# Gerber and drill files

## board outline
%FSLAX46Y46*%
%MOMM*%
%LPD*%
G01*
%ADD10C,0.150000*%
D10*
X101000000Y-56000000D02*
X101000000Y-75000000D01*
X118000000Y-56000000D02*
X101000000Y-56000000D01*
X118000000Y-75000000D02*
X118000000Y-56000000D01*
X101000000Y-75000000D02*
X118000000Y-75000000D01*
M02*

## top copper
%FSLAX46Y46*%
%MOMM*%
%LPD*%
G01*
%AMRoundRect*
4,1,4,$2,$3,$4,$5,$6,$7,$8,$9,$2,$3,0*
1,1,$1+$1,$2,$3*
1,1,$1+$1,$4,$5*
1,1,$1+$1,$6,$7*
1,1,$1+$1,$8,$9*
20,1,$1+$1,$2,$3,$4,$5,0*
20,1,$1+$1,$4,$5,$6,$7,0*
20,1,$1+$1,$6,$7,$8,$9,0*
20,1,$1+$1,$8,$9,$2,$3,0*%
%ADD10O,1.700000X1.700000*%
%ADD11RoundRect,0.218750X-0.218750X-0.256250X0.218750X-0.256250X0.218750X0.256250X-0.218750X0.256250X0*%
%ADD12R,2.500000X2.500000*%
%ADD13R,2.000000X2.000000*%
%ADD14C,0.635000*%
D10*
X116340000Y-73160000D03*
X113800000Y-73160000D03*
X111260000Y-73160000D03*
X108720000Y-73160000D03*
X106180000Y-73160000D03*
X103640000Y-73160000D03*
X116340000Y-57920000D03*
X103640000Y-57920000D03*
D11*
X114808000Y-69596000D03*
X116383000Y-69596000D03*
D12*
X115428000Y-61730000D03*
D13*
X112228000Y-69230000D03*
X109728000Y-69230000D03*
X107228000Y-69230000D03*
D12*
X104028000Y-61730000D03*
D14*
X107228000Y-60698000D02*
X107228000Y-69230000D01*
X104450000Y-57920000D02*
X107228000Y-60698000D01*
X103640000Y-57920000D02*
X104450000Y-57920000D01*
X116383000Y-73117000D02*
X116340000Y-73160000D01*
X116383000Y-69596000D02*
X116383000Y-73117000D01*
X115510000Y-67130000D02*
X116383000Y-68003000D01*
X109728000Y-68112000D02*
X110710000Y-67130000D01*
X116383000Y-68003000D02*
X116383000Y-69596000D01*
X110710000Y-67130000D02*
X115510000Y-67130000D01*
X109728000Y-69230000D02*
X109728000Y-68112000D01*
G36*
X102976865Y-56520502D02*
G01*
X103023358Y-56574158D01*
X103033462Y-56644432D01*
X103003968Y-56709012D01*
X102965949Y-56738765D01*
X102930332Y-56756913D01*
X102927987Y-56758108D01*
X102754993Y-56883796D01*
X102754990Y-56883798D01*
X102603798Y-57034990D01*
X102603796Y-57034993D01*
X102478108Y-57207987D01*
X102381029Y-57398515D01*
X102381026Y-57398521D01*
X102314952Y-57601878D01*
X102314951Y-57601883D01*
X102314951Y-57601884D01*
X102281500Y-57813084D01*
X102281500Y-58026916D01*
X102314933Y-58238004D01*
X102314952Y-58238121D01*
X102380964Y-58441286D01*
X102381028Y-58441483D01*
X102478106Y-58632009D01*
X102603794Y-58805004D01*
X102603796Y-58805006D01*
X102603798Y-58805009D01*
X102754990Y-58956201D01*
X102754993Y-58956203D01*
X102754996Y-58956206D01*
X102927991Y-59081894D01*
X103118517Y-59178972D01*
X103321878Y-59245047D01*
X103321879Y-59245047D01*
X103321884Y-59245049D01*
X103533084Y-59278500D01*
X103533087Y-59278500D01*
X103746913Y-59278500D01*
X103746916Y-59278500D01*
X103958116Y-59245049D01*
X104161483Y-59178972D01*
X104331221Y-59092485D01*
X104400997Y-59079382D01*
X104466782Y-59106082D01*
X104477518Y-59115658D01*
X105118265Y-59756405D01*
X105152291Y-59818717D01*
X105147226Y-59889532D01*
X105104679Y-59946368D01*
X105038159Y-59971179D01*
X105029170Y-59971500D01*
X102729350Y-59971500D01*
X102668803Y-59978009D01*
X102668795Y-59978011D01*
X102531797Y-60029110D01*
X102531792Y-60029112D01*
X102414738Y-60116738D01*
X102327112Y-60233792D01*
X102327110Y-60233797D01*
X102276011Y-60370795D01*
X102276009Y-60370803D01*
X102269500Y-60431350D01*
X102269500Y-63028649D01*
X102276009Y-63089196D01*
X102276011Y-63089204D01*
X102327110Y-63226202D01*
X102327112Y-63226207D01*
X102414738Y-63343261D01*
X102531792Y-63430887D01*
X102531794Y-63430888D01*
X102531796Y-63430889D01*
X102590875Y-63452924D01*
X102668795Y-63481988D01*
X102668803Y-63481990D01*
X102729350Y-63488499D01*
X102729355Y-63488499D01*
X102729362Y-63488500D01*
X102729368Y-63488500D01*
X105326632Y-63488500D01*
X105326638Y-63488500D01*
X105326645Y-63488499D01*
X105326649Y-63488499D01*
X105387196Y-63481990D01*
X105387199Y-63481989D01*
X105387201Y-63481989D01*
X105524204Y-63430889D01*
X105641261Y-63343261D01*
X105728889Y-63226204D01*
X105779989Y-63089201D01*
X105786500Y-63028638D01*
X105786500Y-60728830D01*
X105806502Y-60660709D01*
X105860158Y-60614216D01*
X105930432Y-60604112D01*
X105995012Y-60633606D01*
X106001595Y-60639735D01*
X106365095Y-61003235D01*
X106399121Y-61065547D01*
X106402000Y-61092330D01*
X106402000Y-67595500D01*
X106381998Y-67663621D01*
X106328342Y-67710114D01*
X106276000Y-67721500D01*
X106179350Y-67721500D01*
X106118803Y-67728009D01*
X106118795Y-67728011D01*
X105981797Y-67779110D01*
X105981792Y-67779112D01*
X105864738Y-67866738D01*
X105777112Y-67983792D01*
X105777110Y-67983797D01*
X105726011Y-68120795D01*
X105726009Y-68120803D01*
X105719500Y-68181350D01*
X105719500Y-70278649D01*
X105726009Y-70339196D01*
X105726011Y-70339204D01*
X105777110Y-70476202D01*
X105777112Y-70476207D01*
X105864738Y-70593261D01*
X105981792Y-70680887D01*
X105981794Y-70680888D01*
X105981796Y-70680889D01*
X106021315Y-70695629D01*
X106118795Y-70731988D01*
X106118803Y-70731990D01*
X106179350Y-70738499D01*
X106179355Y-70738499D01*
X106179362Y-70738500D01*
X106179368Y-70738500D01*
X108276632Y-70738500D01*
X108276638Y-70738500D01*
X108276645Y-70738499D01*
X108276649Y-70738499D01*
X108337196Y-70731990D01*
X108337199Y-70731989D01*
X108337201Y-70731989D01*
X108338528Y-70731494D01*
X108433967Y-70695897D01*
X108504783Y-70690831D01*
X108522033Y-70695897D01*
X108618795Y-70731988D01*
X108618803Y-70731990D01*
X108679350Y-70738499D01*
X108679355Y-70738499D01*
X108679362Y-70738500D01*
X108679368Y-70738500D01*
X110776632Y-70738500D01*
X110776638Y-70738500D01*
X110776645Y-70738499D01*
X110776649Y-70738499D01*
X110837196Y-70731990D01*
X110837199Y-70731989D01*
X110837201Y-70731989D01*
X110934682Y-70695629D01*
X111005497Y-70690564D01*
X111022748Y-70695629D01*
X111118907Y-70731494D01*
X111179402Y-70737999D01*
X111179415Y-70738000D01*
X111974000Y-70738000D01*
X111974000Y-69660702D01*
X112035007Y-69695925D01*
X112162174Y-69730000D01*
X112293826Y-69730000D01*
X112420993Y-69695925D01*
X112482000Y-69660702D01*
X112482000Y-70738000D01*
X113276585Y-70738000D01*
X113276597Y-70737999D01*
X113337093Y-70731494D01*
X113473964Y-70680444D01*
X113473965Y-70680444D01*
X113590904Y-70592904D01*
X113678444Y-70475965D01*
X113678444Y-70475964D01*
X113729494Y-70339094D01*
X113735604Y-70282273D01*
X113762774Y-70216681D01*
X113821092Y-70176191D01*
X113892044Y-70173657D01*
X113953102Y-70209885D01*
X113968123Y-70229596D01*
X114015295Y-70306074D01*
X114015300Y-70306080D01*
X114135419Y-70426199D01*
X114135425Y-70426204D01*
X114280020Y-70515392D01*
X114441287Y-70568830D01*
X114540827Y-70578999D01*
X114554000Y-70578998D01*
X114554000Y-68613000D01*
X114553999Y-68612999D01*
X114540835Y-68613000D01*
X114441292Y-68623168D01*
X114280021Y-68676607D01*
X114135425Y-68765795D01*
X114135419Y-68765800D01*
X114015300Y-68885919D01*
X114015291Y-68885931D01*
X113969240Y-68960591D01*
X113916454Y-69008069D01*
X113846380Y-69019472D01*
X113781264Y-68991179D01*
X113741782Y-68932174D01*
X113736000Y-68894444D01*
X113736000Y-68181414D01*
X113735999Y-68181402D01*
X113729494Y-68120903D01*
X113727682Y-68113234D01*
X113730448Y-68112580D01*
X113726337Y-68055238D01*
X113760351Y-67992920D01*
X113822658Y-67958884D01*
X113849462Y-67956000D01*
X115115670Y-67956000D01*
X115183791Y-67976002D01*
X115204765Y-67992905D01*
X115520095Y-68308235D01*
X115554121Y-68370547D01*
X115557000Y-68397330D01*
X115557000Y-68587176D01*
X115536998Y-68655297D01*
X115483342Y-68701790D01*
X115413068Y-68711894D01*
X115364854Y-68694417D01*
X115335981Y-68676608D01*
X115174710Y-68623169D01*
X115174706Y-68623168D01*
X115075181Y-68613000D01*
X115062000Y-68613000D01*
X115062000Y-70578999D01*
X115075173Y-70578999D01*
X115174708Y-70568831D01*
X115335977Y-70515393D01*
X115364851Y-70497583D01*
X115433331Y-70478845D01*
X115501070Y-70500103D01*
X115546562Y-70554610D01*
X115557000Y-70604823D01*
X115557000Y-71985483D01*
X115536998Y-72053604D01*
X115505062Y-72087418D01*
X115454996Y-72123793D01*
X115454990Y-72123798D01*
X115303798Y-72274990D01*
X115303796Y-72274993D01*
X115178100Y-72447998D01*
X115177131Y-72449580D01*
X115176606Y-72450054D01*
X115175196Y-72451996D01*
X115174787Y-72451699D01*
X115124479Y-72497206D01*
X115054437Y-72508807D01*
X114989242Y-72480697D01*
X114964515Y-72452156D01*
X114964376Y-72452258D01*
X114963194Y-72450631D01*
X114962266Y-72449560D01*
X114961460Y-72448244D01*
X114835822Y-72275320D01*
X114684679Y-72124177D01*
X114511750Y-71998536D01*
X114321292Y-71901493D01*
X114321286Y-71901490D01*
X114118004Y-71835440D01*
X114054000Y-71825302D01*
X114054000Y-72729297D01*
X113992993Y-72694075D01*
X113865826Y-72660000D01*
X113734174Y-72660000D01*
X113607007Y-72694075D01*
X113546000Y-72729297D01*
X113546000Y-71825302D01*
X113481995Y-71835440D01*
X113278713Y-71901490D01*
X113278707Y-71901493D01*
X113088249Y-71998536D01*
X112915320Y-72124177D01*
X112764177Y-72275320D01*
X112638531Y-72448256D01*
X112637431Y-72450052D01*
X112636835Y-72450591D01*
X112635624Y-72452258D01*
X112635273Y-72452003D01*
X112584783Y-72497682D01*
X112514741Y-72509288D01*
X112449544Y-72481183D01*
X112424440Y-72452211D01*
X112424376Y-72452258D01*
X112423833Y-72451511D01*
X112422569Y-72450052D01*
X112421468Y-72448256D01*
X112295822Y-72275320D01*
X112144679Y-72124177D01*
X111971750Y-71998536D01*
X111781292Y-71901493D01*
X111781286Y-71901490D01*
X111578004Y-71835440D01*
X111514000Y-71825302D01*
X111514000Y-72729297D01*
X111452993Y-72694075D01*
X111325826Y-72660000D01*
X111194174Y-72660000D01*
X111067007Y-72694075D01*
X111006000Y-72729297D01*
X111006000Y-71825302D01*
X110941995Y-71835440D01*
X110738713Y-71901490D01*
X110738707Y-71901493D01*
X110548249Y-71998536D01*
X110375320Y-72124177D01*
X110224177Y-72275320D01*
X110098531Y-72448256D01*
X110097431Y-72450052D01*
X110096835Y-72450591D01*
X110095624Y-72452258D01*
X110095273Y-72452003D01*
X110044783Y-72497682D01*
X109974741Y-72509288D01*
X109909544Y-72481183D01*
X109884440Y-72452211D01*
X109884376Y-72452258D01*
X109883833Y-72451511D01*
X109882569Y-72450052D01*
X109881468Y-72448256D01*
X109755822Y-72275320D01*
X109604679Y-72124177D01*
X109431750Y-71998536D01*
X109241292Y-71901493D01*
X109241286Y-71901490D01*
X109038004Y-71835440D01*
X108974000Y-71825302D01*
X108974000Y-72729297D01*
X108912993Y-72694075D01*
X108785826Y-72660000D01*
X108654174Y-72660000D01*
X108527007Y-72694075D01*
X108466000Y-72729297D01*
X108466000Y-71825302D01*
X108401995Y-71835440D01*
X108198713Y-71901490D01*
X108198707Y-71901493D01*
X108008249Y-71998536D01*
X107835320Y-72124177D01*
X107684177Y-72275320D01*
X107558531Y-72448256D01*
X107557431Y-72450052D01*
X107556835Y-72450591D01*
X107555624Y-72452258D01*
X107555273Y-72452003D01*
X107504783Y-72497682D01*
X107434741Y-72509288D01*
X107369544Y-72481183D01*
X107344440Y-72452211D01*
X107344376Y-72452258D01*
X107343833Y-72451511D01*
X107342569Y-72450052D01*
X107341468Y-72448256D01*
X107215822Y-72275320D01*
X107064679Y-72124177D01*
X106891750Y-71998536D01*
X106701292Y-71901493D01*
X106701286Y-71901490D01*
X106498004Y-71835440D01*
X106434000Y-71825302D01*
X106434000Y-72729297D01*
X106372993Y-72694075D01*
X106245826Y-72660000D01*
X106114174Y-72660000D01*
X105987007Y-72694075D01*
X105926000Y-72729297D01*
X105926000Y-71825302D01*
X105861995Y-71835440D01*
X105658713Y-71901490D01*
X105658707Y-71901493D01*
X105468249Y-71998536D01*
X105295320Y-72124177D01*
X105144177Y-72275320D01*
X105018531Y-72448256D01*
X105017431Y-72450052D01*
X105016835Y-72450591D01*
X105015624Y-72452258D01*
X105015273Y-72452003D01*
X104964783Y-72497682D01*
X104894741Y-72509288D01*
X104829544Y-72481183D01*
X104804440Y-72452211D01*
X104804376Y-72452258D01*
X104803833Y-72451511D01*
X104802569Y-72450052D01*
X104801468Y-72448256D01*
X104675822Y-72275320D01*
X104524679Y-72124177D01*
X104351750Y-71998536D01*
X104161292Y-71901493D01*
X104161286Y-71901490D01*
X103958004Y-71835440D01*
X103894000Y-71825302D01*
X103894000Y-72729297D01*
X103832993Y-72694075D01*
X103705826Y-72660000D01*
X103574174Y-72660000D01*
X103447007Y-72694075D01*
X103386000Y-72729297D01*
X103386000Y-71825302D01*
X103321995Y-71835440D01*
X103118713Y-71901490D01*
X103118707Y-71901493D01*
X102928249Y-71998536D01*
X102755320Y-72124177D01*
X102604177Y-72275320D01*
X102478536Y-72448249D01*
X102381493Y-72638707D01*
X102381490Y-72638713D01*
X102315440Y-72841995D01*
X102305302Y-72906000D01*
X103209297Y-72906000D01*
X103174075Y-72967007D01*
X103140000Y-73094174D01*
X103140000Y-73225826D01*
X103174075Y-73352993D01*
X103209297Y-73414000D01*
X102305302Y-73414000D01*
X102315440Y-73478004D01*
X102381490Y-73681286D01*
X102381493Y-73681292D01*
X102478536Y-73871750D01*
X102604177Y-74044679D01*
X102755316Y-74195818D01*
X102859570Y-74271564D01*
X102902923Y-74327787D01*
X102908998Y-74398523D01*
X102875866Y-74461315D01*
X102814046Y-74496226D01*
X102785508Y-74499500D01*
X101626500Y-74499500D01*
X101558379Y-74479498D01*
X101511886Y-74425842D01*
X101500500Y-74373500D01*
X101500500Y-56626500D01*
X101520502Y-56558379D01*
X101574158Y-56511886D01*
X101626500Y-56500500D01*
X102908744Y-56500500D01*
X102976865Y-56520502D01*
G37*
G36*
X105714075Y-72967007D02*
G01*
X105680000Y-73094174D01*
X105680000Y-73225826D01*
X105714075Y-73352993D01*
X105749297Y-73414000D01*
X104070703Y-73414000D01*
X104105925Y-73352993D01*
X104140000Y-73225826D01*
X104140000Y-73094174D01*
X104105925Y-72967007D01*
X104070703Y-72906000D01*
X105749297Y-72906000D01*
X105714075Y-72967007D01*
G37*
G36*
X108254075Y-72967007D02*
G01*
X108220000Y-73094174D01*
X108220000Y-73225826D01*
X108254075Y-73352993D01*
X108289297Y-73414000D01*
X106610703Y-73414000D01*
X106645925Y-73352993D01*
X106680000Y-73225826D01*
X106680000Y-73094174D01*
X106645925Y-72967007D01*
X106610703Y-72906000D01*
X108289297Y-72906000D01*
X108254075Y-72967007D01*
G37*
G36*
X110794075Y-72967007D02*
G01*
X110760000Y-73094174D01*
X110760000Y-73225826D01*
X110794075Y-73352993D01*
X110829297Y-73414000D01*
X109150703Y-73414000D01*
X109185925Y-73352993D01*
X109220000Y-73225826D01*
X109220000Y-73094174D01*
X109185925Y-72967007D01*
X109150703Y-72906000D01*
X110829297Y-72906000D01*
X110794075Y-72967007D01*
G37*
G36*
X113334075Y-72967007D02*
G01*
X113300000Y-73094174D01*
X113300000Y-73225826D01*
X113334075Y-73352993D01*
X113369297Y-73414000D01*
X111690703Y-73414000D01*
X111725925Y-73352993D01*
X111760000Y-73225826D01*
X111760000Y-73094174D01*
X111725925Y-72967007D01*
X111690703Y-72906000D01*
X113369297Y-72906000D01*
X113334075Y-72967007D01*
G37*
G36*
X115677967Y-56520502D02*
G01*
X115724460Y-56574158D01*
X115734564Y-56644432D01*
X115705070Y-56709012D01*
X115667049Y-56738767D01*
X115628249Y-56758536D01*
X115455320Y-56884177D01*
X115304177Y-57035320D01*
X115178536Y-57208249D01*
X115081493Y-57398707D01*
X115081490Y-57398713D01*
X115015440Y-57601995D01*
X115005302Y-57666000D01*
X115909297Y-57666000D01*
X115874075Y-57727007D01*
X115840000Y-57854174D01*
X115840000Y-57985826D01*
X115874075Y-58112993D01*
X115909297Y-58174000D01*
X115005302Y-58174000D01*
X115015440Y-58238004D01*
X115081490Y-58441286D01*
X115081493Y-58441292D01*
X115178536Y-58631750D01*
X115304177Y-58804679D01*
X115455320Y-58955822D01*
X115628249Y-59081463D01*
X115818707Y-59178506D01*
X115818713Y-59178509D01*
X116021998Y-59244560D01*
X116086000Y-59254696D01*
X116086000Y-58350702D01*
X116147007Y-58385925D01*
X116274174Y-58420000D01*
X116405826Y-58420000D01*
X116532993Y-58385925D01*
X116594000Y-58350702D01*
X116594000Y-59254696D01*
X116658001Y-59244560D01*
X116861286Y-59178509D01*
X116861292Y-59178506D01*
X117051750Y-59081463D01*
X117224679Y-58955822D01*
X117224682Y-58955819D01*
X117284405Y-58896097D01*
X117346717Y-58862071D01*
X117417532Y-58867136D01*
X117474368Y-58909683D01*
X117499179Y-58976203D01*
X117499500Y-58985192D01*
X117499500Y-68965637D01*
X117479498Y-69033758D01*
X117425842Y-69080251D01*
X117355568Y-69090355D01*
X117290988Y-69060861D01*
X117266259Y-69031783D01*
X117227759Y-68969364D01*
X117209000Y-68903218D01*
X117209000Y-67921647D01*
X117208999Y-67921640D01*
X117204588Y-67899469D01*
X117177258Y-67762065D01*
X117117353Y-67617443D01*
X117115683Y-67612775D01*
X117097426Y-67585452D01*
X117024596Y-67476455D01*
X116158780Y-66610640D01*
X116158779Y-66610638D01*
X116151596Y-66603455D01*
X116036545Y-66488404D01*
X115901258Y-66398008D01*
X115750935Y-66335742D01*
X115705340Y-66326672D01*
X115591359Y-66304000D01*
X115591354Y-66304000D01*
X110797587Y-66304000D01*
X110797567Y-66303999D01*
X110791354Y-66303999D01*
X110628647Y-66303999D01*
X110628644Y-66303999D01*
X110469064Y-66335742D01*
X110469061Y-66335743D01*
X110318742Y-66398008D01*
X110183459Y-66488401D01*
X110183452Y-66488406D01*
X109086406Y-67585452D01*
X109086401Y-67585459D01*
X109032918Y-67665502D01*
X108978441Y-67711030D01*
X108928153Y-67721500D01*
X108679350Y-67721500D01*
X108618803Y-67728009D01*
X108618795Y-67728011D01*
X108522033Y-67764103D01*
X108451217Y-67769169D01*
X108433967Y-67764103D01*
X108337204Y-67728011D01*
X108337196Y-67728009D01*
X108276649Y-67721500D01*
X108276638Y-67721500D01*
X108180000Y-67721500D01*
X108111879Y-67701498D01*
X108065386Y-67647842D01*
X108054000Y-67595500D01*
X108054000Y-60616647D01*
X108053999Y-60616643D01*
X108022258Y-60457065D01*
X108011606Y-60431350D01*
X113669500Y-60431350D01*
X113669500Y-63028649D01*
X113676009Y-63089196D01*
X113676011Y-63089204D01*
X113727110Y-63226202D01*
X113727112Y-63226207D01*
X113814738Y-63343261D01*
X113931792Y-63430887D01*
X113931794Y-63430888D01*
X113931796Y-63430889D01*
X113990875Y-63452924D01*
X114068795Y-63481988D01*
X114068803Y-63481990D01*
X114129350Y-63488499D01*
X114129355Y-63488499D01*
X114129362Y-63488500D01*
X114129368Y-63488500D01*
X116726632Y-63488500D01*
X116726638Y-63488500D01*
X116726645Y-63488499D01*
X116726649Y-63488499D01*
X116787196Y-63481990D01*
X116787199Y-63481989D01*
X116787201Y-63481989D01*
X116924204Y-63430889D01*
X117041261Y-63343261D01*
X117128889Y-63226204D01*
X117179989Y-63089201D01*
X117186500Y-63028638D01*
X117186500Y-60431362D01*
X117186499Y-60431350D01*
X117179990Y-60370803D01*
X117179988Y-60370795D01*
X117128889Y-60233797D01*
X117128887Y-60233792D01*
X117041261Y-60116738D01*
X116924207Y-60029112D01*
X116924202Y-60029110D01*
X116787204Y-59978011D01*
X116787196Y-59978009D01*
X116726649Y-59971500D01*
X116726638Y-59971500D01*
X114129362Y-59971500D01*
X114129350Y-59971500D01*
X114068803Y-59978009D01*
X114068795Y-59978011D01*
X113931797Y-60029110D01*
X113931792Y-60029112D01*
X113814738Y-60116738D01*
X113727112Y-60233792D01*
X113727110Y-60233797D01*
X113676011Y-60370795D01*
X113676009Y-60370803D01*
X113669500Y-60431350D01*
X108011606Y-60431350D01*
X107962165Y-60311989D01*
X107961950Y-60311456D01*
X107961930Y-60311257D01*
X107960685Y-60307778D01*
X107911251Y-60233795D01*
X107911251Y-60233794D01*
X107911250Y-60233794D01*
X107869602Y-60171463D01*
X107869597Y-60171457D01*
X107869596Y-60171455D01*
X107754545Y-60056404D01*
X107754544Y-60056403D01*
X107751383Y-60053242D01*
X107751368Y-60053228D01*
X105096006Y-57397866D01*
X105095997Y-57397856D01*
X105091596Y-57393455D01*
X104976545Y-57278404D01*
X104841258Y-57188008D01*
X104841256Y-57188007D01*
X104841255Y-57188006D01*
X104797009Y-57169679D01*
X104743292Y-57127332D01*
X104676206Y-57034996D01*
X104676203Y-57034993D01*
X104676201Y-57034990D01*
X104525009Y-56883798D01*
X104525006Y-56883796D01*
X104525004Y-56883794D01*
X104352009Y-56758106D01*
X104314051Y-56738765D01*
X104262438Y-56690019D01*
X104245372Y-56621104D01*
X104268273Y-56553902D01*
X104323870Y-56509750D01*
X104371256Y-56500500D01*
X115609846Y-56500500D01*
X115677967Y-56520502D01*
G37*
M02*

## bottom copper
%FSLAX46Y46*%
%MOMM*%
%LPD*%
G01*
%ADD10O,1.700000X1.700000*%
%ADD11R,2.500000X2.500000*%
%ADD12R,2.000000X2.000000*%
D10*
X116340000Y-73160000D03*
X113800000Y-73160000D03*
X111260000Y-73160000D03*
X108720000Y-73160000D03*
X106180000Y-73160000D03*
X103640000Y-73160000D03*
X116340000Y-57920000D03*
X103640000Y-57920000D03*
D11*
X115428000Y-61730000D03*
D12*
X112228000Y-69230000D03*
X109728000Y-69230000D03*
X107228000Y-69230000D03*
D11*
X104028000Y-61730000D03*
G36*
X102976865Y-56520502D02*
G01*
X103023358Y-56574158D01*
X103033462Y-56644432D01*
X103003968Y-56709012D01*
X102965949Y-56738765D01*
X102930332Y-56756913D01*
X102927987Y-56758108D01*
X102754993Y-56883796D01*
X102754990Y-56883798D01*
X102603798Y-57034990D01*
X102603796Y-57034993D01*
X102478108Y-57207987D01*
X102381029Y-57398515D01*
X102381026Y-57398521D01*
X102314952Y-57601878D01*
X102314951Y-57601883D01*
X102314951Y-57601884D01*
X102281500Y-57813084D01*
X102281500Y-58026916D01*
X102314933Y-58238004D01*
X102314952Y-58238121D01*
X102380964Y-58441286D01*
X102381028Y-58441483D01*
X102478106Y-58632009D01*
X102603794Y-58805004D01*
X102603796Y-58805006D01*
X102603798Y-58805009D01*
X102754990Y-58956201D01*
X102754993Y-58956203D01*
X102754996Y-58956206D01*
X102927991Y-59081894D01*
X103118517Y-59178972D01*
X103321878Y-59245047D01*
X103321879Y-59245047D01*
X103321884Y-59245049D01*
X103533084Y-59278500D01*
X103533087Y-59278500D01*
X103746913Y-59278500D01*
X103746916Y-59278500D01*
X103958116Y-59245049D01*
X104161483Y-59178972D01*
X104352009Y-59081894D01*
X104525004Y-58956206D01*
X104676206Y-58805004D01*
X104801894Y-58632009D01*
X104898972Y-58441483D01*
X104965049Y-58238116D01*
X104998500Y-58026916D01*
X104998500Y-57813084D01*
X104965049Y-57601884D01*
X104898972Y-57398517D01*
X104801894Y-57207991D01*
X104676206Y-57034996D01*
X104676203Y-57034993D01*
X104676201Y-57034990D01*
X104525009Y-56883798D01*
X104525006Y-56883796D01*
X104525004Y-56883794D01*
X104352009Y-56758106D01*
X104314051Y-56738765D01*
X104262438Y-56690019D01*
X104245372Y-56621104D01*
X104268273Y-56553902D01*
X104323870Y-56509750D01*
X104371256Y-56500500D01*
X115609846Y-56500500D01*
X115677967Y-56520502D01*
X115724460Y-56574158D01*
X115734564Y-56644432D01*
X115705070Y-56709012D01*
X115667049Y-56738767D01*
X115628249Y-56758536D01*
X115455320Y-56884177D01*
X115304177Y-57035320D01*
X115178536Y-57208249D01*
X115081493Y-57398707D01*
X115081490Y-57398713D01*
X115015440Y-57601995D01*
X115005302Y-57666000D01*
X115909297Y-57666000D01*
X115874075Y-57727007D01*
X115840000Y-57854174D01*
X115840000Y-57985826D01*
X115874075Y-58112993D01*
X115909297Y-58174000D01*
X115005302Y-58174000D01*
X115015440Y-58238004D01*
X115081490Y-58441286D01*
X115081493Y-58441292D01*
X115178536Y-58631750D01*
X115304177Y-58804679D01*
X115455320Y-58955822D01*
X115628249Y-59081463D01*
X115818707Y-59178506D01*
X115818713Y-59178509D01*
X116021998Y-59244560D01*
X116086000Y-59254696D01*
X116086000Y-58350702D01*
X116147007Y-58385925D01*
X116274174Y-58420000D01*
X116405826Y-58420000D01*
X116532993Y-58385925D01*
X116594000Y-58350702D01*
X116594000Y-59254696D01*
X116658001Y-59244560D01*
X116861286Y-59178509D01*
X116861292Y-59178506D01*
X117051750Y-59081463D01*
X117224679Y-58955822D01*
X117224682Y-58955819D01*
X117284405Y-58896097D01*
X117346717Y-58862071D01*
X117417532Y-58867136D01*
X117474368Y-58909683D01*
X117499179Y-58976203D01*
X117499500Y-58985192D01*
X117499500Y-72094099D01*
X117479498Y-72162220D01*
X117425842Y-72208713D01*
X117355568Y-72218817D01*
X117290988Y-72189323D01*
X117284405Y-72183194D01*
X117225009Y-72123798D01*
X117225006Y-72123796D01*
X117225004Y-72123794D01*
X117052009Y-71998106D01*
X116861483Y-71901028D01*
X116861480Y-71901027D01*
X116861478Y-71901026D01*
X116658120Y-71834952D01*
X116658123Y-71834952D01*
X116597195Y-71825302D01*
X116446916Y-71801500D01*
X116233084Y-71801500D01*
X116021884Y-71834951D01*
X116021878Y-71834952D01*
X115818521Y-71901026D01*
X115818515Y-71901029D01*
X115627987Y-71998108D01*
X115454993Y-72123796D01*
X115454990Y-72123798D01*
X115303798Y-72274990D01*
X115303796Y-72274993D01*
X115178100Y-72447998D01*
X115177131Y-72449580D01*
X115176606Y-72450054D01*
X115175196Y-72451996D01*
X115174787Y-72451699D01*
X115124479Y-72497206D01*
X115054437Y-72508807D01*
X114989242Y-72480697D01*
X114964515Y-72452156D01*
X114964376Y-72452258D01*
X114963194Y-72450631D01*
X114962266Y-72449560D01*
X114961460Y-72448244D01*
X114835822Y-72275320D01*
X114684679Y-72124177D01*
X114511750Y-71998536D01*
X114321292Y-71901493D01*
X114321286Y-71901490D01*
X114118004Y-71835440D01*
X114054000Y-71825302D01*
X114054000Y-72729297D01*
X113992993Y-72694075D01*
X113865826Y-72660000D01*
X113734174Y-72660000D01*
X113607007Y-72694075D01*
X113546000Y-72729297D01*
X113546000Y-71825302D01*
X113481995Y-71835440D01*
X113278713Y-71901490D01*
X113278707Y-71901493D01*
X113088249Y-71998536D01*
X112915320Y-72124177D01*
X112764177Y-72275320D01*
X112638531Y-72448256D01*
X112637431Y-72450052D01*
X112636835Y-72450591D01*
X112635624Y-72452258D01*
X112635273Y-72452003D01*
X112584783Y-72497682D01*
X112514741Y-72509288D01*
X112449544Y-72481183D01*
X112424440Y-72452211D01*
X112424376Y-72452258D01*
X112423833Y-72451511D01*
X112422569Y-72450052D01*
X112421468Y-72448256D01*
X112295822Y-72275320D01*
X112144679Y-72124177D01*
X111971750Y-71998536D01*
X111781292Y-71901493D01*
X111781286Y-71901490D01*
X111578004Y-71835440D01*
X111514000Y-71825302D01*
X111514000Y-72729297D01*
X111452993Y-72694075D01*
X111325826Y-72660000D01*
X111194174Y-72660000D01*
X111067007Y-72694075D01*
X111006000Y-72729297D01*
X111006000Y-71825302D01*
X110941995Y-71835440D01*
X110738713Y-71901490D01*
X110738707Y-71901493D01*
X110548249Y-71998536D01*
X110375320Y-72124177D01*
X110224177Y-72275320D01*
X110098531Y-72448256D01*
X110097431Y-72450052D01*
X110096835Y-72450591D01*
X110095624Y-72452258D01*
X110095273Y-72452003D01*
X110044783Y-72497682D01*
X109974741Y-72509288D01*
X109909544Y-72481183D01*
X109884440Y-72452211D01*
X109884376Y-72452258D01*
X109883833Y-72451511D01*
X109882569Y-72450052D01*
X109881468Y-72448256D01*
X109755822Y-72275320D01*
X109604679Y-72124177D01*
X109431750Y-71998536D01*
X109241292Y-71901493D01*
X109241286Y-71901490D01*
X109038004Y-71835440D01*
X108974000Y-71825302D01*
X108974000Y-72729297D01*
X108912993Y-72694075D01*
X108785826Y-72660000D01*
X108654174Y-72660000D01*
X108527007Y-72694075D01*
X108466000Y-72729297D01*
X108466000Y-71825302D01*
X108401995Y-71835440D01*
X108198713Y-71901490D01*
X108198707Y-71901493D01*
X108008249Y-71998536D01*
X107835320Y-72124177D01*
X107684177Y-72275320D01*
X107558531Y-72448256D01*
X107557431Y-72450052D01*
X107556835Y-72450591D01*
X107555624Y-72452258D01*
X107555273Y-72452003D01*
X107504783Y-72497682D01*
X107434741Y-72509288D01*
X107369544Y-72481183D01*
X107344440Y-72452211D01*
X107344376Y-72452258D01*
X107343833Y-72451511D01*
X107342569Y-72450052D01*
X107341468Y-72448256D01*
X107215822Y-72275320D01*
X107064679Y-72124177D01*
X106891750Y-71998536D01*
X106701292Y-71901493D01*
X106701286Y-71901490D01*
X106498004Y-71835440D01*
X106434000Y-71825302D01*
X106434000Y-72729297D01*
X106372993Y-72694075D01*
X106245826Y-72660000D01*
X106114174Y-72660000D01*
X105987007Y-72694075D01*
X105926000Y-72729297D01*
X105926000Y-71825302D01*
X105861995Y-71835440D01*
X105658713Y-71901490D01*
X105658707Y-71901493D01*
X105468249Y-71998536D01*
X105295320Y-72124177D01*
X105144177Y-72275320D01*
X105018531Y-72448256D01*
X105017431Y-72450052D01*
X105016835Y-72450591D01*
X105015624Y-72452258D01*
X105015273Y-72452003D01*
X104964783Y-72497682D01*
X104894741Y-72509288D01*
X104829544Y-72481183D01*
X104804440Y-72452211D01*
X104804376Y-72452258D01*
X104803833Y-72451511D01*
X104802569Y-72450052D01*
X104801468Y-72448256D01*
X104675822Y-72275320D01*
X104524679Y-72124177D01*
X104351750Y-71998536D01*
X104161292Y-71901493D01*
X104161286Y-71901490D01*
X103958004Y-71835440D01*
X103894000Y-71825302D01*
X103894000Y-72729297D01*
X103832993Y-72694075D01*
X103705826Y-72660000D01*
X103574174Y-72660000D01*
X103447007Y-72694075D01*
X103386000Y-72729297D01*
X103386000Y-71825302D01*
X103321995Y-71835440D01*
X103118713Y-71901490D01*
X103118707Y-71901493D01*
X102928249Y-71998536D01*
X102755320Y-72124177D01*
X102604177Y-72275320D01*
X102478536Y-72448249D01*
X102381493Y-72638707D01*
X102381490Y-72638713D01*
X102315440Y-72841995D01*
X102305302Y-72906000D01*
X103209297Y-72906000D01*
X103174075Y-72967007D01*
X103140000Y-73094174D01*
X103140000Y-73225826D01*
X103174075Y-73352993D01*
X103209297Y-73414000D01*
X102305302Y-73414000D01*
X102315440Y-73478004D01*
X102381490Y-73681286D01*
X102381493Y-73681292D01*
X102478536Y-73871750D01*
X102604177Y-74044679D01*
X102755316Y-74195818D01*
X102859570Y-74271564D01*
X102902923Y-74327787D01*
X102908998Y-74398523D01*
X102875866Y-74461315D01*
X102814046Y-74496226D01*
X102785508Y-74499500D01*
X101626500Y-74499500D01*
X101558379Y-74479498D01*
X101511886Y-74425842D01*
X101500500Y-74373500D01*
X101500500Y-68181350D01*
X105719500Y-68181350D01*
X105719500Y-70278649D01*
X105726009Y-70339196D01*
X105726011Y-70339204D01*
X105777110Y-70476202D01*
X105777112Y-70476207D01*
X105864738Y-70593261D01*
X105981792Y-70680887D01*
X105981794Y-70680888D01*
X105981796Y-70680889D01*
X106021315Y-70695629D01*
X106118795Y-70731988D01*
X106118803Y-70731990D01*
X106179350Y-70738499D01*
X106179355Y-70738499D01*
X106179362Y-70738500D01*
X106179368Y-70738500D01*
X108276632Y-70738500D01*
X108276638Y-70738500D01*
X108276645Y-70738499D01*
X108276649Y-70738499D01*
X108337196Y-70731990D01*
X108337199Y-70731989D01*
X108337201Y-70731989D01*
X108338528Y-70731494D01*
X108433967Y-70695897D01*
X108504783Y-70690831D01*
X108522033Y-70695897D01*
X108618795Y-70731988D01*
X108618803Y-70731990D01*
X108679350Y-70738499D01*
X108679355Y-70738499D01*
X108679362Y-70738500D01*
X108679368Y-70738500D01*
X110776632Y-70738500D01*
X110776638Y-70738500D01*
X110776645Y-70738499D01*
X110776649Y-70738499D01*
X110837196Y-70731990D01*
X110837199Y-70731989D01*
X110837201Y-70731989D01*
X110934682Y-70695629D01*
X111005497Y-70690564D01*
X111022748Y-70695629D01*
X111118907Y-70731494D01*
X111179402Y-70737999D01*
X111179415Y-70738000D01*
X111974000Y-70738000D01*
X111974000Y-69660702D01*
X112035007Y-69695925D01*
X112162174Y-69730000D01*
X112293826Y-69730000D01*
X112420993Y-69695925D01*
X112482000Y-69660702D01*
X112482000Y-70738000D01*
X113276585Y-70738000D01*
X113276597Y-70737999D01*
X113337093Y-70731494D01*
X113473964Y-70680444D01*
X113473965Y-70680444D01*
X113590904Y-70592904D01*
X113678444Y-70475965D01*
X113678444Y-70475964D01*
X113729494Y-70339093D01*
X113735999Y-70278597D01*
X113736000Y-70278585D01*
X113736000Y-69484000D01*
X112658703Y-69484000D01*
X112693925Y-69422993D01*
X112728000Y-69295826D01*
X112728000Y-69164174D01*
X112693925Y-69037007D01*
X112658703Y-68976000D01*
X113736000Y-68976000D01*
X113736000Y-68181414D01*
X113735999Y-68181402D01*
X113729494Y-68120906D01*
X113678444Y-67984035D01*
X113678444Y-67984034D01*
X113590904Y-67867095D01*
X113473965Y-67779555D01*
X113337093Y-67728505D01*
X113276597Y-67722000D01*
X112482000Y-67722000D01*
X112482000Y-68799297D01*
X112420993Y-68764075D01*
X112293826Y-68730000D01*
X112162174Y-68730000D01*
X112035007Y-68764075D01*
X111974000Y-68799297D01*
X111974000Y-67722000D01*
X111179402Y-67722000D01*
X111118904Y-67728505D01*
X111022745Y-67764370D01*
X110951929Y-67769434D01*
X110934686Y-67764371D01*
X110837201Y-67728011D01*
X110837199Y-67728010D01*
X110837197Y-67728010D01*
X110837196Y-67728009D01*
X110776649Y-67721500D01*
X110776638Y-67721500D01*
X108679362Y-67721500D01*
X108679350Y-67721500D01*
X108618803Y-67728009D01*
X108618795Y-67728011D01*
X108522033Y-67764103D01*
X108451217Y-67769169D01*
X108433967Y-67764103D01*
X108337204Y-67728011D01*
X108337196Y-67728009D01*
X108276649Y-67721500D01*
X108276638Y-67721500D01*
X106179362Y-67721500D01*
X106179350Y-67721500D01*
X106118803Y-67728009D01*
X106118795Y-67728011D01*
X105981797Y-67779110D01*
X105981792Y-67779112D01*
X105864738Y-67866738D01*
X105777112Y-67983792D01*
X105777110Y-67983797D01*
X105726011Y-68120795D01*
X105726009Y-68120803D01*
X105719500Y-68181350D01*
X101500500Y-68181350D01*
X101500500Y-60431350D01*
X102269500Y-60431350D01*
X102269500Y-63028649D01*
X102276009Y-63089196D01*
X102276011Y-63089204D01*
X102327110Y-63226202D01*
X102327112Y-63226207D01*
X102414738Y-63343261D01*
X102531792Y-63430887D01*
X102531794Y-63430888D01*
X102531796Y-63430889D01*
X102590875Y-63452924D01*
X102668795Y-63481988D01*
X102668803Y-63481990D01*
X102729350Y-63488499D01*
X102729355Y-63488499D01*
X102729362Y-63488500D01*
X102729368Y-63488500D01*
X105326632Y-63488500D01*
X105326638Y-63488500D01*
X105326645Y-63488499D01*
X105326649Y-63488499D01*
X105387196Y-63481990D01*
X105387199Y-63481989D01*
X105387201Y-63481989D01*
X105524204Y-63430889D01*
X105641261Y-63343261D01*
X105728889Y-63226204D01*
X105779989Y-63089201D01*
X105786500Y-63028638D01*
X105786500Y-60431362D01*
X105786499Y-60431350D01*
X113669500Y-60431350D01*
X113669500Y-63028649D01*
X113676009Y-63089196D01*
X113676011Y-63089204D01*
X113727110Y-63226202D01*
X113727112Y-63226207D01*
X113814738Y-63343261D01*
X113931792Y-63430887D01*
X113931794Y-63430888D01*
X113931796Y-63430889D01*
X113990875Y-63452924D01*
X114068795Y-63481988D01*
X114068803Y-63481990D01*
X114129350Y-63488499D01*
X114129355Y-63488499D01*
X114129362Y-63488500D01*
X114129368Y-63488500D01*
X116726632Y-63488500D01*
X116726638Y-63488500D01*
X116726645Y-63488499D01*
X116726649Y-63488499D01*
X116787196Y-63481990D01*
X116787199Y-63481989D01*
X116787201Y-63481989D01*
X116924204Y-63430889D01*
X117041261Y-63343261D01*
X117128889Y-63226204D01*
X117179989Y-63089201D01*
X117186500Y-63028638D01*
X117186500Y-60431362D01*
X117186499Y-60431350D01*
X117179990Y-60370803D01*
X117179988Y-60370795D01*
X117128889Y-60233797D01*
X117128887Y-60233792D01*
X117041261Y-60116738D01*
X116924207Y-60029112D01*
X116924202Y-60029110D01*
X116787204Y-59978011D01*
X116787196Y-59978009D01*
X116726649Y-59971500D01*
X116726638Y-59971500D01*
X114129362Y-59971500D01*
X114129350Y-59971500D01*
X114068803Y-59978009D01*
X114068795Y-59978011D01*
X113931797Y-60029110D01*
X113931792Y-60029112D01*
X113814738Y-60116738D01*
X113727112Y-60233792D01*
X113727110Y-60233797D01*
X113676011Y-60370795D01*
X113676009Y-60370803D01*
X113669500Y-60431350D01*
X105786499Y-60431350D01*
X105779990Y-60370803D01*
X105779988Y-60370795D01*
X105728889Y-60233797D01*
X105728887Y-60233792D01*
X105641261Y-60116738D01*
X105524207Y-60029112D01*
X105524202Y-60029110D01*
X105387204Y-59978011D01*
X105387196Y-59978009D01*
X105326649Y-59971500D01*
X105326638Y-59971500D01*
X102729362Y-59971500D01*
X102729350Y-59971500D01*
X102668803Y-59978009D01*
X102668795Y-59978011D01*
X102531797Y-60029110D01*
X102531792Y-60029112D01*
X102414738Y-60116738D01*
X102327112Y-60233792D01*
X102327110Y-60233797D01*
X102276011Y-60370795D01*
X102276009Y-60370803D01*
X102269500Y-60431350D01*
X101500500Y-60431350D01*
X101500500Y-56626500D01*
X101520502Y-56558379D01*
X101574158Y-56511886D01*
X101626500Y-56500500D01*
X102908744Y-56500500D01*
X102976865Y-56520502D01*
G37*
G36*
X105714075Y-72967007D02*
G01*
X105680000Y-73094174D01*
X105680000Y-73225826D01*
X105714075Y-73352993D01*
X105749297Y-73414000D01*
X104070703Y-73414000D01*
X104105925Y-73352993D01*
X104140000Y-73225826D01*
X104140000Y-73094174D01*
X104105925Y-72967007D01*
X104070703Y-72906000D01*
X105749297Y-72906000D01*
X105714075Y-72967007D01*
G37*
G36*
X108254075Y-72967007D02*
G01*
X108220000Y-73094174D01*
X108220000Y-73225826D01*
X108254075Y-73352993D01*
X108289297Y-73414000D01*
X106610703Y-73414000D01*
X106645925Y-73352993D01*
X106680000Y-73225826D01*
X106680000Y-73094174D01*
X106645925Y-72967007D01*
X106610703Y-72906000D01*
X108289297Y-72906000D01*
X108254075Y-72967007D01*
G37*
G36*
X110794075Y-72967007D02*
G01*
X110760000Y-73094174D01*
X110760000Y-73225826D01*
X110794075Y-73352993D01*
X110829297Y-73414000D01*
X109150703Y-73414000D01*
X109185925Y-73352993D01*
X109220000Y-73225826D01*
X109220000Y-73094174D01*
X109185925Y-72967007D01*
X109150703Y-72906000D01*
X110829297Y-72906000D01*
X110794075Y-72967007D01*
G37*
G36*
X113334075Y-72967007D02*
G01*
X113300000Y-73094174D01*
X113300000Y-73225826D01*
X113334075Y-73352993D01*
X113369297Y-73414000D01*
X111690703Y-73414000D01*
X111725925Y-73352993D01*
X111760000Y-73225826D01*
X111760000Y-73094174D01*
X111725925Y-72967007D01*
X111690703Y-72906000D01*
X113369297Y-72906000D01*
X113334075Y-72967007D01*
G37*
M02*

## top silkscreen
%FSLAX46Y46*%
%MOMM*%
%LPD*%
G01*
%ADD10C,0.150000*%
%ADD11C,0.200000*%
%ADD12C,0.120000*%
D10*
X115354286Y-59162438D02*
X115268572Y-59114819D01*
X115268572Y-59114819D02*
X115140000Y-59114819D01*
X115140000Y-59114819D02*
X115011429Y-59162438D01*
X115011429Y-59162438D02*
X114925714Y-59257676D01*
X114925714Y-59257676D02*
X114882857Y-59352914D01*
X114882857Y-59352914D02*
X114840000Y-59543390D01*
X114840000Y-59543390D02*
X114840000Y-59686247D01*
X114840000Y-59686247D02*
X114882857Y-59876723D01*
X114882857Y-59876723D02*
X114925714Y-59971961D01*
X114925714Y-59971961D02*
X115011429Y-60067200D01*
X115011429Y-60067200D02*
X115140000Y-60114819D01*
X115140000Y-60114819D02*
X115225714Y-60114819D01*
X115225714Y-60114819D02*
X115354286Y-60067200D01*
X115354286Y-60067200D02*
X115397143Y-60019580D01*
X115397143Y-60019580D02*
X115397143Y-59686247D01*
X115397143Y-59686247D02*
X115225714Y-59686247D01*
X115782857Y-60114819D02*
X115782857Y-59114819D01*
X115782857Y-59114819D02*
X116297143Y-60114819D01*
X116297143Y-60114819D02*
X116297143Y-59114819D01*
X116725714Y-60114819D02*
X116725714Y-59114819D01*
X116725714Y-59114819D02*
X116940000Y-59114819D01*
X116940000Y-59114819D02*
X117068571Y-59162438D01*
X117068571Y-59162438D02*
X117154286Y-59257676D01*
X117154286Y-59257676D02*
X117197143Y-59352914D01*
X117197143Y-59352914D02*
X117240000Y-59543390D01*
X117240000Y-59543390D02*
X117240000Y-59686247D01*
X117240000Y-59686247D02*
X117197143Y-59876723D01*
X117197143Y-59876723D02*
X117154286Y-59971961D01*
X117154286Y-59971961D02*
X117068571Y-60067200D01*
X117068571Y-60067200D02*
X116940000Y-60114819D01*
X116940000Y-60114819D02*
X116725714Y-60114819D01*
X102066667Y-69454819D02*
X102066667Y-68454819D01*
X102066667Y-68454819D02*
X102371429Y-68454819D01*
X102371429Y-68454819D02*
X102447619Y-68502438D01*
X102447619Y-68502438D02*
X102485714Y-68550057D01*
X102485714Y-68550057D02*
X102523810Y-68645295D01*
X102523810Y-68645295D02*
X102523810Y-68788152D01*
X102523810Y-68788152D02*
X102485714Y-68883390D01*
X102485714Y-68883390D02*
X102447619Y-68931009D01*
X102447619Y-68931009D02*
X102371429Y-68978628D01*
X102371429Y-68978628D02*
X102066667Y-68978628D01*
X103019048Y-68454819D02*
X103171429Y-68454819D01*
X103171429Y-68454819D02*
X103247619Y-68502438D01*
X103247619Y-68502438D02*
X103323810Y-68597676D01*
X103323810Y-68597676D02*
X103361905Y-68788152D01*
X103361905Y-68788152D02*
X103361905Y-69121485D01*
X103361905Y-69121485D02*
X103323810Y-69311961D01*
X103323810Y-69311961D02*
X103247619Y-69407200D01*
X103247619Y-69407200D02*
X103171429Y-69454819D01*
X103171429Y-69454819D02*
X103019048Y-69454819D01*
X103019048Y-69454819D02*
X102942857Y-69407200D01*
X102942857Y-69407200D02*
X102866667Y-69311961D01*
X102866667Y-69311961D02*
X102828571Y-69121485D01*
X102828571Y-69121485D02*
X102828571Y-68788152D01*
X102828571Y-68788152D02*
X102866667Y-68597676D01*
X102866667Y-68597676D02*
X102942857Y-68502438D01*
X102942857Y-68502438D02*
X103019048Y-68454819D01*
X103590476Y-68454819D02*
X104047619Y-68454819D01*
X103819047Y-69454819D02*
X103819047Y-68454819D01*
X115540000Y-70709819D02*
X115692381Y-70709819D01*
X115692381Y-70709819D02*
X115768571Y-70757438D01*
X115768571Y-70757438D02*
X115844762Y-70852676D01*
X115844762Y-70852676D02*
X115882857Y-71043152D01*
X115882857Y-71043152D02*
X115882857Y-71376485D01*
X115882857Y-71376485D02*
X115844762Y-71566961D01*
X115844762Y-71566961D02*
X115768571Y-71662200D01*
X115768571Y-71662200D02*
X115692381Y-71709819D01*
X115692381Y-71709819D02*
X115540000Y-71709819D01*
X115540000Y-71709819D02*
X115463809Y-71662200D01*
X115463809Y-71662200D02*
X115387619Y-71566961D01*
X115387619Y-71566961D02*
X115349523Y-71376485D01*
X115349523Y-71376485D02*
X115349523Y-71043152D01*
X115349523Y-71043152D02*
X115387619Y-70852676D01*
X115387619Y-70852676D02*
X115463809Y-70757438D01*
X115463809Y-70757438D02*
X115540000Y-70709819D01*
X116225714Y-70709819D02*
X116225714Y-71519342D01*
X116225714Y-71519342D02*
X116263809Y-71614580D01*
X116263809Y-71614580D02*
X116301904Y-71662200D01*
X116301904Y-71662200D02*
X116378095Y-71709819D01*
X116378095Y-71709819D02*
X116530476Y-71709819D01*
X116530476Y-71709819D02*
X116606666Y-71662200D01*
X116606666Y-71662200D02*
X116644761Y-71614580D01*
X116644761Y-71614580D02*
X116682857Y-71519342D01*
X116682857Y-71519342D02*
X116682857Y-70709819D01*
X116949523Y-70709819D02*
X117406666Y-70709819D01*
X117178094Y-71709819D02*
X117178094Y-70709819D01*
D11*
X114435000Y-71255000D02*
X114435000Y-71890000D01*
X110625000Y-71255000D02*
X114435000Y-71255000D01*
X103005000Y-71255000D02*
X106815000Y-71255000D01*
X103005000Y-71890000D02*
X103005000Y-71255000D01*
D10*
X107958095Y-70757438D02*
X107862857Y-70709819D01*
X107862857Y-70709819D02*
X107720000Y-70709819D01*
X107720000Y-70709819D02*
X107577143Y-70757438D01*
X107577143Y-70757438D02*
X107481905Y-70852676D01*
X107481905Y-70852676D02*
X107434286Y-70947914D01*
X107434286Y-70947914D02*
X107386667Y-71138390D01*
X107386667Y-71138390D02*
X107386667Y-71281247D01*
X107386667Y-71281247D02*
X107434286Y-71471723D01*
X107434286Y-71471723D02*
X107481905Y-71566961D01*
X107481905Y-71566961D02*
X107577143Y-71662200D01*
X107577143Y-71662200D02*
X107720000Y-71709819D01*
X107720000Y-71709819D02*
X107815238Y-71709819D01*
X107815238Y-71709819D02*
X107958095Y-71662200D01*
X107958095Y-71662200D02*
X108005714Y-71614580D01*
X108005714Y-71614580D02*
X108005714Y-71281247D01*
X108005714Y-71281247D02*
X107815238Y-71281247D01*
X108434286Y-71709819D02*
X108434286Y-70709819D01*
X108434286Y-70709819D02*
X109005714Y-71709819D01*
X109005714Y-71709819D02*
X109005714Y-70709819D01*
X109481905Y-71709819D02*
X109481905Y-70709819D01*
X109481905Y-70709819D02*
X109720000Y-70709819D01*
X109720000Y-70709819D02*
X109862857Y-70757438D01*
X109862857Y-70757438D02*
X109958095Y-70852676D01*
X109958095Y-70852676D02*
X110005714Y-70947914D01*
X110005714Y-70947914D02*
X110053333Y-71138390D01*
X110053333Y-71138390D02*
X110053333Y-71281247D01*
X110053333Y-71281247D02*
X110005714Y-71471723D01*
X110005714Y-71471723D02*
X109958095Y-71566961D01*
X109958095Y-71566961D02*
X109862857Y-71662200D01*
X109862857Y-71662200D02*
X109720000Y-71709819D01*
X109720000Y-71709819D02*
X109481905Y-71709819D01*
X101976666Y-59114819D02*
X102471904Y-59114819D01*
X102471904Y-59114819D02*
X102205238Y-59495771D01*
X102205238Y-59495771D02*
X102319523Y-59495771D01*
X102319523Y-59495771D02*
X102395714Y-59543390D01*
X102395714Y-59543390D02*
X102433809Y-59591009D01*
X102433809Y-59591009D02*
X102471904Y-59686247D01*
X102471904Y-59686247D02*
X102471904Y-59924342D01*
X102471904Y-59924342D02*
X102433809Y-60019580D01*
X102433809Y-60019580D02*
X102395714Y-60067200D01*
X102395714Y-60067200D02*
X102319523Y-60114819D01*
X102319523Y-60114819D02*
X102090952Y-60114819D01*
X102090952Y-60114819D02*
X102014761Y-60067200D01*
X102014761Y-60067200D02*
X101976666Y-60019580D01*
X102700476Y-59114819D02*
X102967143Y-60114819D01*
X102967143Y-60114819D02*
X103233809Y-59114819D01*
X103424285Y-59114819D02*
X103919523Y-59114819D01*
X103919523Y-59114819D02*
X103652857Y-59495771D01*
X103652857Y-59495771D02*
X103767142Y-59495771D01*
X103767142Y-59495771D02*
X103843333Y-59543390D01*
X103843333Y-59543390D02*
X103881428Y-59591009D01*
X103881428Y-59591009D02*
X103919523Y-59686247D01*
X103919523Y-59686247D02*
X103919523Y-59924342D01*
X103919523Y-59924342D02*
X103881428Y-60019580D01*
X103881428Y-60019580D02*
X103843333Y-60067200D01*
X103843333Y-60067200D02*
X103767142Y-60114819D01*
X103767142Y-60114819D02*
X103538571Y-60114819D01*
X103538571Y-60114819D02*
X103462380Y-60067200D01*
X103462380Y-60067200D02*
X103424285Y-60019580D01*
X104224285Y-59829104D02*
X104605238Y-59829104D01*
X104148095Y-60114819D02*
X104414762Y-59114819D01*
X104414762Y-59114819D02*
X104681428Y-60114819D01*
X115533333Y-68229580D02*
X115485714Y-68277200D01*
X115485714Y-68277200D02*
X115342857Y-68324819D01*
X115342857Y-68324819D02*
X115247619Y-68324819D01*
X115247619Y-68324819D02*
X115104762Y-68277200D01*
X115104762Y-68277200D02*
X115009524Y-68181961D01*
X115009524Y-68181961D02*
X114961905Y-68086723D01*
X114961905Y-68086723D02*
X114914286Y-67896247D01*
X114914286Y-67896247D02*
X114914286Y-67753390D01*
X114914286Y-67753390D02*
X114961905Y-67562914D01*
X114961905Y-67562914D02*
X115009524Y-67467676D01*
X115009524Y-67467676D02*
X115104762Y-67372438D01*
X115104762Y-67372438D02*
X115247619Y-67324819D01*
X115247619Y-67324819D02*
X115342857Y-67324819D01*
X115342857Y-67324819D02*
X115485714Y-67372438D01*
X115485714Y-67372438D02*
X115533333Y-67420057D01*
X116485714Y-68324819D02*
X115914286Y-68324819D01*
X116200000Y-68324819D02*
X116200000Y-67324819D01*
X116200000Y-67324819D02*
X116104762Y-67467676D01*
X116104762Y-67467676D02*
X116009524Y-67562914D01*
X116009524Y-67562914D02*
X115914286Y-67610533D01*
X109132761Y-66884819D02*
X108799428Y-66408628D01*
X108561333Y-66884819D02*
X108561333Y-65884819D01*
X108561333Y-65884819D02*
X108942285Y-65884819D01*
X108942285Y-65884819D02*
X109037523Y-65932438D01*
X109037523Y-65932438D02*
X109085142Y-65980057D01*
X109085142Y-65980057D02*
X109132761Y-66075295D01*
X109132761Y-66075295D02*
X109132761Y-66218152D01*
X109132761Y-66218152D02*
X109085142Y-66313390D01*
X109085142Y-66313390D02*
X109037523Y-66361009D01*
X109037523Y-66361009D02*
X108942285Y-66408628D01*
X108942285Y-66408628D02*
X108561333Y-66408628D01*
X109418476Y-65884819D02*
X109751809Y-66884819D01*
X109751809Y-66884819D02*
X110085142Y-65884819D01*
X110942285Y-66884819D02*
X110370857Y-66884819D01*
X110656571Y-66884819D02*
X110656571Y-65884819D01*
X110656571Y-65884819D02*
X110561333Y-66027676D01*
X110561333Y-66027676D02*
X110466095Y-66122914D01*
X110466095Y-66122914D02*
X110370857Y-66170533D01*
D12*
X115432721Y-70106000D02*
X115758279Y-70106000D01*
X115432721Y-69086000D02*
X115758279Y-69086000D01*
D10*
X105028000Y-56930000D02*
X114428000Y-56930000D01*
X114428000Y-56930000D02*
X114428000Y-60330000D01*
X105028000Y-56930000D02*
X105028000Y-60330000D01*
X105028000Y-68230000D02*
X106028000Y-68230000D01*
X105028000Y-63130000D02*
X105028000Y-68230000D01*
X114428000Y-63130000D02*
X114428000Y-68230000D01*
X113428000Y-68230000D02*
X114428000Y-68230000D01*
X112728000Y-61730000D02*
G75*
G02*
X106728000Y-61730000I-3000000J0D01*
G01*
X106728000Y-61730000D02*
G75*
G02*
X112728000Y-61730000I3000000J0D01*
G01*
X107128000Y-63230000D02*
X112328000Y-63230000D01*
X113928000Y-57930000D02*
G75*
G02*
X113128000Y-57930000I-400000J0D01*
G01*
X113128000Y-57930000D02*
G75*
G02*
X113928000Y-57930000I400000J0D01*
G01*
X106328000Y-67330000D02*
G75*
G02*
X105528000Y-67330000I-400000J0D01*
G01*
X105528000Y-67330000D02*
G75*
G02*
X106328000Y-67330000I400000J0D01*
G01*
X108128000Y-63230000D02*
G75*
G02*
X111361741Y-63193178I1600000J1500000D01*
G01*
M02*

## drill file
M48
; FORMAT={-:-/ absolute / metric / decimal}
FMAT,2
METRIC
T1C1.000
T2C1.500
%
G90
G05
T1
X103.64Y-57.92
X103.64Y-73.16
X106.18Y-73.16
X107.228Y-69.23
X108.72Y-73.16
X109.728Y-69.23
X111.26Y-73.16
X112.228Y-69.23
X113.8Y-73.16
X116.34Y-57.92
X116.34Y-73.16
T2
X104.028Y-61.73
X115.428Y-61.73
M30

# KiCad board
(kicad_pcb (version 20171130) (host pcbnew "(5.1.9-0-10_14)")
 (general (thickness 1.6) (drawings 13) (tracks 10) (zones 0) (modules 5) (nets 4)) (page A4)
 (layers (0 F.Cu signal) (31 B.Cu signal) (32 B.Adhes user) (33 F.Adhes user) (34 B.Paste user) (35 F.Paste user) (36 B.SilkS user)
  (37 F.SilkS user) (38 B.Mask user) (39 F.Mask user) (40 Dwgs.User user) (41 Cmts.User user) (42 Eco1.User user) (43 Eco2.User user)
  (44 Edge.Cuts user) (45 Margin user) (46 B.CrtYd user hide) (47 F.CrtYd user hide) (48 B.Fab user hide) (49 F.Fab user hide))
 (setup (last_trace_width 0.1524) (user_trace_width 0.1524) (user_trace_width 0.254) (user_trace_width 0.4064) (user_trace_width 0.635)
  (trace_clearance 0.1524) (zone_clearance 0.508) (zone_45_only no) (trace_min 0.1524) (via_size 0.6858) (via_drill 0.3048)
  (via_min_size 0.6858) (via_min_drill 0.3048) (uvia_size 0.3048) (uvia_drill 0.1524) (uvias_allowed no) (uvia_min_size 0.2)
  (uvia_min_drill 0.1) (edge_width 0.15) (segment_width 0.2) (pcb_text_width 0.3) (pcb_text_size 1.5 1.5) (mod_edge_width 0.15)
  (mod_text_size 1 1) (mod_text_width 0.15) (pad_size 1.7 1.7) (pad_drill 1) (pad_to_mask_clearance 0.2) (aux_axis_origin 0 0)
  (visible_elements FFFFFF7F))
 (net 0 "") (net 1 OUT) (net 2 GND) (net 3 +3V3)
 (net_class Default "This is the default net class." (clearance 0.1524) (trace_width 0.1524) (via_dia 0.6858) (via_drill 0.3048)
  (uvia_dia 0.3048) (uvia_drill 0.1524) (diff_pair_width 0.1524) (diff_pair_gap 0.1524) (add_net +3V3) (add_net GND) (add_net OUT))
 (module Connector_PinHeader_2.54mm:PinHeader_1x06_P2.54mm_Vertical (layer B.Cu) (at 116.34 73.16 90)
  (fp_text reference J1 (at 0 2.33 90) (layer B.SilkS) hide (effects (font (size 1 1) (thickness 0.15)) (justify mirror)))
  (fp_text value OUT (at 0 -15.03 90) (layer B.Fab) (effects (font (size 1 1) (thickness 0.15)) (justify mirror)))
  (pad 1 thru_hole oval (at 0 0 90) (size 1.7 1.7) (drill 1) (layers *.Cu *.Mask) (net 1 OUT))
  (pad 2 thru_hole oval (at 0 -2.54 90) (size 1.7 1.7) (drill 1) (layers *.Cu *.Mask) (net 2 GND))
  (pad 3 thru_hole oval (at 0 -5.08 90) (size 1.7 1.7) (drill 1) (layers *.Cu *.Mask) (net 2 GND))
  (pad 4 thru_hole oval (at 0 -7.62 90) (size 1.7 1.7) (drill 1) (layers *.Cu *.Mask) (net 2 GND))
  (pad 5 thru_hole oval (at 0 -10.16 90) (size 1.7 1.7) (drill 1) (layers *.Cu *.Mask) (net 2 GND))
  (pad 6 thru_hole oval (at 0 -12.7 90) (size 1.7 1.7) (drill 1) (layers *.Cu *.Mask) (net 2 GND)))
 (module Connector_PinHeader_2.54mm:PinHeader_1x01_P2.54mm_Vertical (layer B.Cu) (at 116.34 57.92 90)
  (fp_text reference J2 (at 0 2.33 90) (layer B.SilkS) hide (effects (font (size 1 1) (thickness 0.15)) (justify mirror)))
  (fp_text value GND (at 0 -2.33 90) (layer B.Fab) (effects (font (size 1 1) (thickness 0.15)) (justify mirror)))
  (pad 1 thru_hole oval (at 0 0 90) (size 1.7 1.7) (drill 1) (layers *.Cu *.Mask) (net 2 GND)))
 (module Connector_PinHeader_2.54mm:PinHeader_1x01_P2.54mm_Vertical (layer B.Cu) (at 103.64 57.92 270)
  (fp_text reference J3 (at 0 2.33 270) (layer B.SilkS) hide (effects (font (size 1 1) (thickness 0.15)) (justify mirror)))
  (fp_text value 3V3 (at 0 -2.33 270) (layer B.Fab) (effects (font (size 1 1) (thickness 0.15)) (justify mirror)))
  (pad 1 thru_hole oval (at 0 0 270) (size 1.7 1.7) (drill 1) (layers *.Cu *.Mask) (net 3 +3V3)))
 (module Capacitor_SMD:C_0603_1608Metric (layer F.Cu) (at 115.5955 69.596)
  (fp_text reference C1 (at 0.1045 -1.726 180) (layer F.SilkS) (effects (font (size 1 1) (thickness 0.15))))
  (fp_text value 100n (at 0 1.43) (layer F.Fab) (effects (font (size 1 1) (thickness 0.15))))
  (fp_line (start -0.162779 0.51) (end 0.162779 0.51) (layer F.SilkS) (width 0.12))
  (fp_line (start -0.162779 -0.51) (end 0.162779 -0.51) (layer F.SilkS) (width 0.12))
  (pad 1 smd roundrect (at -0.7875 0) (size 0.875 0.95) (layers F.Cu F.Paste F.Mask) (roundrect_rratio 0.25) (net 2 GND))
  (pad 2 smd roundrect (at 0.7875 0) (size 0.875 0.95) (layers F.Cu F.Paste F.Mask) (roundrect_rratio 0.25) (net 1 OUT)))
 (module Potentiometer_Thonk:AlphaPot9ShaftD (layer F.Cu) (at 109.728 61.73)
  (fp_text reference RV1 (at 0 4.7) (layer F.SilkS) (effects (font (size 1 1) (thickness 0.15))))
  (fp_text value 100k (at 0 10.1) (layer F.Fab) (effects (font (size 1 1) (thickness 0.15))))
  (fp_line (start -4.7 -4.8) (end 4.7 -4.8) (layer F.SilkS) (width 0.15))
  (fp_line (start 4.7 -4.8) (end 4.7 -1.4) (layer F.SilkS) (width 0.15))
  (fp_line (start -4.7 -4.8) (end -4.7 -1.4) (layer F.SilkS) (width 0.15))
  (fp_line (start -4.7 6.5) (end -3.7 6.5) (layer F.SilkS) (width 0.15))
  (fp_line (start -4.7 1.4) (end -4.7 6.5) (layer F.SilkS) (width 0.15))
  (fp_line (start 4.7 1.4) (end 4.7 6.5) (layer F.SilkS) (width 0.15))
  (fp_line (start 3.7 6.5) (end 4.7 6.5) (layer F.SilkS) (width 0.15))
  (fp_circle (center 0 0) (end 3 0) (layer F.SilkS) (width 0.15))
  (fp_line (start -2.6 1.5) (end 2.6 1.5) (layer F.SilkS) (width 0.15))
  (fp_circle (center 3.8 -3.8) (end 4.2 -3.8) (layer F.SilkS) (width 0.15))
  (fp_circle (center -3.8 5.6) (end -4.2 5.6) (layer F.SilkS) (width 0.15))
  (fp_arc (start 0 0) (end -1.6 1.5) (angle 265) (layer F.SilkS) (width 0.15))
  (pad "" thru_hole rect (at 5.7 0) (size 2.5 2.5) (drill 1.5) (layers *.Cu *.Mask))
  (pad 3 thru_hole rect (at 2.5 7.5) (size 2 2) (drill 1) (layers *.Cu *.Mask) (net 2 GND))
  (pad 2 thru_hole rect (at 0 7.5) (size 2 2) (drill 1) (layers *.Cu *.Mask) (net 1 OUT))
  (pad 1 thru_hole rect (at -2.5 7.5) (size 2 2) (drill 1) (layers *.Cu *.Mask) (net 3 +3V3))
  (pad "" thru_hole rect (at -5.7 0) (size 2.5 2.5) (drill 1.5) (layers *.Cu *.Mask)))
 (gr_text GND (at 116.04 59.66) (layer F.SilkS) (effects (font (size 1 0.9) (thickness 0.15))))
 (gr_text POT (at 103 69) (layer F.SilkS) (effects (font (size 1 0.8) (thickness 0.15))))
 (gr_line (start 101 56) (end 101 75) (layer Edge.Cuts) (width 0.15))
 (gr_line (start 118 56) (end 101 56) (layer Edge.Cuts) (width 0.15))
 (gr_line (start 118 75) (end 118 56) (layer Edge.Cuts) (width 0.15))
 (gr_line (start 101 75) (end 118 75) (layer Edge.Cuts) (width 0.15))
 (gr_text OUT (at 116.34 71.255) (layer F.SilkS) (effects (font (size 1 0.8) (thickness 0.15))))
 (gr_line (start 114.435 71.255) (end 114.435 71.89) (layer F.SilkS) (width 0.2))
 (gr_line (start 110.625 71.255) (end 114.435 71.255) (layer F.SilkS) (width 0.2))
 (gr_line (start 103.005 71.255) (end 106.815 71.255) (layer F.SilkS) (width 0.2))
 (gr_line (start 103.005 71.89) (end 103.005 71.255) (layer F.SilkS) (width 0.2))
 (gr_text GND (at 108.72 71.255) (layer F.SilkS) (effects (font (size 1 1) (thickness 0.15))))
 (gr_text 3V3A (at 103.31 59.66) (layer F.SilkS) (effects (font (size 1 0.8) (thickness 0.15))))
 (segment (start 107.228 60.698) (end 107.228 69.23) (width 0.635) (layer F.Cu) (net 3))
 (segment (start 104.45 57.92) (end 107.228 60.698) (width 0.635) (layer F.Cu) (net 3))
 (segment (start 103.64 57.92) (end 104.45 57.92) (width 0.635) (layer F.Cu) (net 3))
 (segment (start 116.383 73.117) (end 116.34 73.16) (width 0.635) (layer F.Cu) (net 1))
 (segment (start 116.383 69.596) (end 116.383 73.117) (width 0.635) (layer F.Cu) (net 1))
 (segment (start 115.51 67.13) (end 116.383 68.003) (width 0.635) (layer F.Cu) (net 1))
 (segment (start 109.728 68.112) (end 110.71 67.13) (width 0.635) (layer F.Cu) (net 1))
 (segment (start 116.383 68.003) (end 116.383 69.596) (width 0.635) (layer F.Cu) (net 1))
 (segment (start 110.71 67.13) (end 115.51 67.13) (width 0.635) (layer F.Cu) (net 1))
 (segment (start 109.728 69.23) (end 109.728 68.112) (width 0.635) (layer F.Cu) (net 1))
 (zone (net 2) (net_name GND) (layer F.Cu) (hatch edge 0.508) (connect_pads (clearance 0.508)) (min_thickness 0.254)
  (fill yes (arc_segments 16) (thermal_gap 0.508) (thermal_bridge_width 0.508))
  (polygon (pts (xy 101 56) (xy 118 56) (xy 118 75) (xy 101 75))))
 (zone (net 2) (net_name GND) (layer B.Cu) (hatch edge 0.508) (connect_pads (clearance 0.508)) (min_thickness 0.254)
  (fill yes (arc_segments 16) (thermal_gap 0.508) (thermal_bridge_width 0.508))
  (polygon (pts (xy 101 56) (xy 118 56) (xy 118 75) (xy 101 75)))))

